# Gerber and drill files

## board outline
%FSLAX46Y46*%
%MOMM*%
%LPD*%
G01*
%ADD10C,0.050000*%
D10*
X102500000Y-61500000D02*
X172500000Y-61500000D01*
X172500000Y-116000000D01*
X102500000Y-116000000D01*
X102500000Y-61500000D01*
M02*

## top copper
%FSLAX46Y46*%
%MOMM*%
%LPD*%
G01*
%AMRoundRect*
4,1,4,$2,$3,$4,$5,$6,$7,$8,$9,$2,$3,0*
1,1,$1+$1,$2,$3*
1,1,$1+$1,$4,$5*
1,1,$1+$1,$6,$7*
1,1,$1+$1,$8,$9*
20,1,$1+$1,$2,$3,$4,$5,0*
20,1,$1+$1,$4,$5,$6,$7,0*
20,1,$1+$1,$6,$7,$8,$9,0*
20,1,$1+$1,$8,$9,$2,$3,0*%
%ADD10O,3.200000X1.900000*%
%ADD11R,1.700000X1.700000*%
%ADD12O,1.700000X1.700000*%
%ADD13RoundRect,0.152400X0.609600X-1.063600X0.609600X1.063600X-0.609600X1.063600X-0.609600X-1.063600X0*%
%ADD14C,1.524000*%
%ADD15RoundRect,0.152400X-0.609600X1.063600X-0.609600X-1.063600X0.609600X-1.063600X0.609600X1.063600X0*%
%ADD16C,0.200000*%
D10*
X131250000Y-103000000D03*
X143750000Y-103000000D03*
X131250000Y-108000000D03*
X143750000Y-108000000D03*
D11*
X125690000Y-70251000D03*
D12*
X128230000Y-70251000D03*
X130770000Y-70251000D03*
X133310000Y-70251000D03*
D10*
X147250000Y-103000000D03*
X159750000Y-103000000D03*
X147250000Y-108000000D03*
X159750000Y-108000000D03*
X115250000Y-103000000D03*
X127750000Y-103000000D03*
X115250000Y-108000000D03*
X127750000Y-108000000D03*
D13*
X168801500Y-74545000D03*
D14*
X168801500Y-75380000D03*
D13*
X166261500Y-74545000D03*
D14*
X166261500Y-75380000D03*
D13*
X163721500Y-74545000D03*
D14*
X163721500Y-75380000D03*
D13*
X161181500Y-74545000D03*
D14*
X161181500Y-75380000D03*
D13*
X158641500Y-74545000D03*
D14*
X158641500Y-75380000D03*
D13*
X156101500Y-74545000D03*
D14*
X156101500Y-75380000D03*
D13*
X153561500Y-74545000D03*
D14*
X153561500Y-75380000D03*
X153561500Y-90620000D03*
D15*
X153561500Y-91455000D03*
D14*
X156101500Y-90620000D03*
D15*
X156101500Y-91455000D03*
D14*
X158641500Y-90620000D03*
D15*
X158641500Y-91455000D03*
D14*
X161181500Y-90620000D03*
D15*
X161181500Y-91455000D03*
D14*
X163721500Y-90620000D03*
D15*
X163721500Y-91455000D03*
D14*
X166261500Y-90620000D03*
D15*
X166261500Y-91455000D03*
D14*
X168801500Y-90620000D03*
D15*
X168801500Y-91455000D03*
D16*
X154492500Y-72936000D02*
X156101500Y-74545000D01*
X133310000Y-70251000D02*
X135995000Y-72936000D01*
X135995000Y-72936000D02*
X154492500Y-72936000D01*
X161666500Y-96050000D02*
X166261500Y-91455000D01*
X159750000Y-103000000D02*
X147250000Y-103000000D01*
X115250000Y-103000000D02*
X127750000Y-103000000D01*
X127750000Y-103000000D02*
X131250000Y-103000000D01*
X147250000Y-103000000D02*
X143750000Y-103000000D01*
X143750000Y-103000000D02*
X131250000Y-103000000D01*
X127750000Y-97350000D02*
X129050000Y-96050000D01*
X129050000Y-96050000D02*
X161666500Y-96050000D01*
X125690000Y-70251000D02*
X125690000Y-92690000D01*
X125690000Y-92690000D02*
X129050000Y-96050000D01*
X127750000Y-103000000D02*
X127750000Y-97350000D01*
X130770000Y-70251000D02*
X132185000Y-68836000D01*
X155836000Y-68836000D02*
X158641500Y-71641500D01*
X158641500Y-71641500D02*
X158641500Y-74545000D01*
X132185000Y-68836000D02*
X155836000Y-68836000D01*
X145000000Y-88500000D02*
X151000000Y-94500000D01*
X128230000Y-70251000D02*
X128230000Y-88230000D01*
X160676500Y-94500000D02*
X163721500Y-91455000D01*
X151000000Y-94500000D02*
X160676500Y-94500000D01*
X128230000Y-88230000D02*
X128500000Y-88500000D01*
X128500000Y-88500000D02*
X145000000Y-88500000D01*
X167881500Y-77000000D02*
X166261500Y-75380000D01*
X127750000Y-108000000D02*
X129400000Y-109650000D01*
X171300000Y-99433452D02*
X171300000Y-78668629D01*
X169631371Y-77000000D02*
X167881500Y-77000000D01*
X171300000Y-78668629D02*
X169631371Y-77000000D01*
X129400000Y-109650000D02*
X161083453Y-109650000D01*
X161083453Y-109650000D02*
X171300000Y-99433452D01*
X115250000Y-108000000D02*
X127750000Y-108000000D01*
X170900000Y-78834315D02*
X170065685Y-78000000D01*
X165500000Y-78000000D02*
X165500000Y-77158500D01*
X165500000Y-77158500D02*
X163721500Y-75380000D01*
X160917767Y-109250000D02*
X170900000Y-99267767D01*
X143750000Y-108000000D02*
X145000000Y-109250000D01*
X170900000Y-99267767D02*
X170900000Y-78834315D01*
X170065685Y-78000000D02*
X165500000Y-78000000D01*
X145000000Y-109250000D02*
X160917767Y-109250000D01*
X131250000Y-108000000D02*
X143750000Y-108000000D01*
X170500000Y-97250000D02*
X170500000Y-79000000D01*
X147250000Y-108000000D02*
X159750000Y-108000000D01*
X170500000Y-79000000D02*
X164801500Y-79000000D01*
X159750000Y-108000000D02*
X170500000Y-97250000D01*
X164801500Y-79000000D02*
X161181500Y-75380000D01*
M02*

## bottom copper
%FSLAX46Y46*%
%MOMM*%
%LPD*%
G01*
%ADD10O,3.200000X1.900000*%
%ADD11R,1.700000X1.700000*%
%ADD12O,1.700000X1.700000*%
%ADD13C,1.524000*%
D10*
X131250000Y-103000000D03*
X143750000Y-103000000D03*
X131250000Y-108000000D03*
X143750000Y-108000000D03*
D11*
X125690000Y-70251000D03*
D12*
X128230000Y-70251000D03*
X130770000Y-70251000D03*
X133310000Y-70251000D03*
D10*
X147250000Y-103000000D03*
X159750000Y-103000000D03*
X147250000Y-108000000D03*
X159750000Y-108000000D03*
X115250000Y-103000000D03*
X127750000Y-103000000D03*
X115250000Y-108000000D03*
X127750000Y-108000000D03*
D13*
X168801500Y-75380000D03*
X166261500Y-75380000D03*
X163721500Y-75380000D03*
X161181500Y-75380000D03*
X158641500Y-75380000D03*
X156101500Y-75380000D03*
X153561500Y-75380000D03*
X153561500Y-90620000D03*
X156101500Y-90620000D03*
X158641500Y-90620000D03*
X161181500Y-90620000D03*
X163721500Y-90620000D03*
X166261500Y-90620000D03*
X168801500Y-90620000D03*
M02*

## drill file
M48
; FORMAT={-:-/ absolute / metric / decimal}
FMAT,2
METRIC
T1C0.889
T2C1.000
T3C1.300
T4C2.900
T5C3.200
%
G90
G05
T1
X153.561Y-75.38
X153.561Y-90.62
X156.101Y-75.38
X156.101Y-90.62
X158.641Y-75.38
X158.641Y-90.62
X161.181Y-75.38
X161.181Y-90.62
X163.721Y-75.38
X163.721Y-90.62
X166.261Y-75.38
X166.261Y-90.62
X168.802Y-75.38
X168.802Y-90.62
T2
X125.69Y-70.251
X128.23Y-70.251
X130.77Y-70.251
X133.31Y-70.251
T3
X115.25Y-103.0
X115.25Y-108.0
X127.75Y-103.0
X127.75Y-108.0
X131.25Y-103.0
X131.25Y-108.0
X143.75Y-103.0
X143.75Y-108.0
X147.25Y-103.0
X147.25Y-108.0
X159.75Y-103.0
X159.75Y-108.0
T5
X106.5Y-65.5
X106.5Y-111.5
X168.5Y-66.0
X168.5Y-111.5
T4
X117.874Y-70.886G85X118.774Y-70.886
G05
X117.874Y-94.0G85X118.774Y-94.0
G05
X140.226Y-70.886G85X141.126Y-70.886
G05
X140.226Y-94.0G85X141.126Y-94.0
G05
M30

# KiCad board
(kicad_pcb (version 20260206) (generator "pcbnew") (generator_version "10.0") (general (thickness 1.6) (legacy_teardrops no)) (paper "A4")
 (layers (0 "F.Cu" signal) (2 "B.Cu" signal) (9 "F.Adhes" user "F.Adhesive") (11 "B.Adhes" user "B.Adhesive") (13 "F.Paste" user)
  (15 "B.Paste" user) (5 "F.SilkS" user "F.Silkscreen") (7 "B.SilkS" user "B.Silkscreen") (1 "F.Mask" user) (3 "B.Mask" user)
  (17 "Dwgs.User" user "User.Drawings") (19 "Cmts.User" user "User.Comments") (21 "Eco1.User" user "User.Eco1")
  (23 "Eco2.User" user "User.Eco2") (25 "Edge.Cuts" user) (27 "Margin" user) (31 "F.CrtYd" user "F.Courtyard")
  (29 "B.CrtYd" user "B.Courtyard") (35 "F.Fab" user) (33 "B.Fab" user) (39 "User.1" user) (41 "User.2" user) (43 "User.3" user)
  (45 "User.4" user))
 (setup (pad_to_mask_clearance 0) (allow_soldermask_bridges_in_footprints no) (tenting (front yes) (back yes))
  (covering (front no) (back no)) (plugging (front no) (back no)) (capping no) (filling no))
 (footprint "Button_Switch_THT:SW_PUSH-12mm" (layer "F.Cu") (at 131.25 103)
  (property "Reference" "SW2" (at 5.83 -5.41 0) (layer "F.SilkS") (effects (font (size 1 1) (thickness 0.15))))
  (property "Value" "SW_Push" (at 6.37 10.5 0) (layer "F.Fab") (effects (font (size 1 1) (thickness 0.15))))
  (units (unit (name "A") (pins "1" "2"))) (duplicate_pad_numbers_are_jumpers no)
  (pad "1" thru_hole oval (at 0 0) (size 3.2 1.9) (drill 1.3) (layers "*.Cu" "*.Mask") (remove_unused_layers no) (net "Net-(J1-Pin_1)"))
  (pad "1" thru_hole oval (at 12.5 0) (size 3.2 1.9) (drill 1.3) (layers "*.Cu" "*.Mask") (remove_unused_layers no) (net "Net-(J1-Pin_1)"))
  (pad "2" thru_hole oval (at 0 5) (size 3.2 1.9) (drill 1.3) (layers "*.Cu" "*.Mask") (remove_unused_layers no) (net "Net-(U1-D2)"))
  (pad "2" thru_hole oval (at 12.5 5) (size 3.2 1.9) (drill 1.3) (layers "*.Cu" "*.Mask") (remove_unused_layers no) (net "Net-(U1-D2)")))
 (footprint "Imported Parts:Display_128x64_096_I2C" (layer "F.Cu") (at 129.5 70.251)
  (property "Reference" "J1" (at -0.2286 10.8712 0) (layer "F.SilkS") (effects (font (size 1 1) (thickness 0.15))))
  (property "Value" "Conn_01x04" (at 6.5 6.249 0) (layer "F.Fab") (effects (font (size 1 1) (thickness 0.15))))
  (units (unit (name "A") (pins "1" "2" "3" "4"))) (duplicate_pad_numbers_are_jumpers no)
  (pad "" np_thru_hole oval (at -11.176 0.635) (size 3.8 2.9) (drill oval 3.8 2.9) (layers "*.Cu" "*.Mask"))
  (pad "" np_thru_hole oval (at -11.176 23.749) (size 3.8 2.9) (drill oval 3.8 2.9) (layers "*.Cu" "*.Mask"))
  (pad "" np_thru_hole oval (at 11.176 0.635) (size 3.8 2.9) (drill oval 3.8 2.9) (layers "*.Cu" "*.Mask"))
  (pad "" np_thru_hole oval (at 11.176 23.749) (size 3.8 2.9) (drill oval 3.8 2.9) (layers "*.Cu" "*.Mask"))
  (pad "1" thru_hole rect (at -3.81 0 90) (size 1.7 1.7) (drill 1) (layers "*.Cu" "*.Mask") (remove_unused_layers no) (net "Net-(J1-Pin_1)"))
  (pad "2" thru_hole oval (at -1.27 0 90) (size 1.7 1.7) (drill 1) (layers "*.Cu" "*.Mask") (remove_unused_layers no) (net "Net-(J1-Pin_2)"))
  (pad "3" thru_hole oval (at 1.27 0 90) (size 1.7 1.7) (drill 1) (layers "*.Cu" "*.Mask") (remove_unused_layers no) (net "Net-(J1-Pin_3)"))
  (pad "4" thru_hole oval (at 3.81 0 90) (size 1.7 1.7) (drill 1) (layers "*.Cu" "*.Mask") (remove_unused_layers no) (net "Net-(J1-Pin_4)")))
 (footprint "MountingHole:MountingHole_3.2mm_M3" (layer "F.Cu") (at 168.5 66)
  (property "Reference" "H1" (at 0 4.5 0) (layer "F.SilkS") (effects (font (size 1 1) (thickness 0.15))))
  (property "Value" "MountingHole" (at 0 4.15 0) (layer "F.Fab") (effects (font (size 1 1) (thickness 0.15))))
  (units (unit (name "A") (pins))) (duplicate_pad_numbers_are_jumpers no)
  (pad "" np_thru_hole circle (at 0 0) (size 3.2 3.2) (drill 3.2) (layers "*.Cu" "*.Mask")))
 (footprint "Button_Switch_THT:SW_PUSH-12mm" (layer "F.Cu") (at 147.25 103)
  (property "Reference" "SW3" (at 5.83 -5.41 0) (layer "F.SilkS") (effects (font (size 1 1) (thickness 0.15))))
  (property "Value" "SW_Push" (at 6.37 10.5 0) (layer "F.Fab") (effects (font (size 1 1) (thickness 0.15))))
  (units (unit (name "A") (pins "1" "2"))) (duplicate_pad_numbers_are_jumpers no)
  (pad "1" thru_hole oval (at 0 0) (size 3.2 1.9) (drill 1.3) (layers "*.Cu" "*.Mask") (remove_unused_layers no) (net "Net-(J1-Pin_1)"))
  (pad "1" thru_hole oval (at 12.5 0) (size 3.2 1.9) (drill 1.3) (layers "*.Cu" "*.Mask") (remove_unused_layers no) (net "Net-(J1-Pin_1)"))
  (pad "2" thru_hole oval (at 0 5) (size 3.2 1.9) (drill 1.3) (layers "*.Cu" "*.Mask") (remove_unused_layers no) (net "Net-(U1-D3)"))
  (pad "2" thru_hole oval (at 12.5 5) (size 3.2 1.9) (drill 1.3) (layers "*.Cu" "*.Mask") (remove_unused_layers no) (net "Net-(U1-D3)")))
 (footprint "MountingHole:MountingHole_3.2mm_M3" (layer "F.Cu") (at 168.5 111.5)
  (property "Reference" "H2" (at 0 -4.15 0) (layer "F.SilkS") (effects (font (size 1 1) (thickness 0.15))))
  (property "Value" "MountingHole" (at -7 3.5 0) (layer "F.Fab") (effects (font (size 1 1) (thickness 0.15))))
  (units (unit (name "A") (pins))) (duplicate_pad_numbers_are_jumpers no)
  (pad "" np_thru_hole circle (at 0 0) (size 3.2 3.2) (drill 3.2) (layers "*.Cu" "*.Mask")))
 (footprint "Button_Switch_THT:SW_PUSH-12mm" (layer "F.Cu") (at 115.25 103)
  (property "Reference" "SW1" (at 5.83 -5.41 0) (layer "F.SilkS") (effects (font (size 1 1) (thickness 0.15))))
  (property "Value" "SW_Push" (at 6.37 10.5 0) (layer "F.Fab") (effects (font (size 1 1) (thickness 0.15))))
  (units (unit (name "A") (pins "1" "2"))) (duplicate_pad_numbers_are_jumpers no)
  (pad "1" thru_hole oval (at 0 0) (size 3.2 1.9) (drill 1.3) (layers "*.Cu" "*.Mask") (remove_unused_layers no) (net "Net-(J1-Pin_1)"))
  (pad "1" thru_hole oval (at 12.5 0) (size 3.2 1.9) (drill 1.3) (layers "*.Cu" "*.Mask") (remove_unused_layers no) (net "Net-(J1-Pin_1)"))
  (pad "2" thru_hole oval (at 0 5) (size 3.2 1.9) (drill 1.3) (layers "*.Cu" "*.Mask") (remove_unused_layers no) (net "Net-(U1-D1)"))
  (pad "2" thru_hole oval (at 12.5 5) (size 3.2 1.9) (drill 1.3) (layers "*.Cu" "*.Mask") (remove_unused_layers no) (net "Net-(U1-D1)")))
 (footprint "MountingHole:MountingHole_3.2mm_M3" (layer "F.Cu") (at 106.5 65.5)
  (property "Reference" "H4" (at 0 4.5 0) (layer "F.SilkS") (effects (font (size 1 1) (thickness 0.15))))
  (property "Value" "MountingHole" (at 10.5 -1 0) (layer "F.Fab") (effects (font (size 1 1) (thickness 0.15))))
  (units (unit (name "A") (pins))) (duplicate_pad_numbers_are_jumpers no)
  (pad "" np_thru_hole circle (at 0 0) (size 3.2 3.2) (drill 3.2) (layers "*.Cu" "*.Mask")))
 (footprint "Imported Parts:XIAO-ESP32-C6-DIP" (layer "F.Cu") (at 161.1815 83)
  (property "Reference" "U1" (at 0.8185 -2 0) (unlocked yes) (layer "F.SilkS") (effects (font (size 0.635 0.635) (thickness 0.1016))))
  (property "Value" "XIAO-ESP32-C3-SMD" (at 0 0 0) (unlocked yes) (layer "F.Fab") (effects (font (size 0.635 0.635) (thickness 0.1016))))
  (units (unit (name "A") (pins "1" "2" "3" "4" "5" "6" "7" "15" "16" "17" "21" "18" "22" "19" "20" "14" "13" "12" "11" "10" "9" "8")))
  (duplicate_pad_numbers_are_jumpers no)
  (pad "1" smd roundrect (at 7.62 -8.455 90) (size 2.432 1.524) (layers "F.Cu" "F.Mask") (roundrect_rratio 0.1)
   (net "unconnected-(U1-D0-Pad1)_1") (thermal_bridge_angle 45))
  (pad "1" thru_hole circle (at 7.62 -7.62 90) (size 1.524 1.524) (drill 0.889) (layers "*.Cu" "*.Mask") (remove_unused_layers no)
   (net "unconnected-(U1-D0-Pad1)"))
  (pad "2" smd roundrect (at 5.08 -8.455 90) (size 2.432 1.524) (layers "F.Cu" "F.Mask") (roundrect_rratio 0.1) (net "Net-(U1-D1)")
   (thermal_bridge_angle 45))
  (pad "2" thru_hole circle (at 5.08 -7.62 90) (size 1.524 1.524) (drill 0.889) (layers "*.Cu" "*.Mask") (remove_unused_layers no)
   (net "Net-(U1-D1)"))
  (pad "3" smd roundrect (at 2.54 -8.455 90) (size 2.432 1.524) (layers "F.Cu" "F.Mask") (roundrect_rratio 0.1) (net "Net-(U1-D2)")
   (thermal_bridge_angle 45))
  (pad "3" thru_hole circle (at 2.54 -7.62 90) (size 1.524 1.524) (drill 0.889) (layers "*.Cu" "*.Mask") (remove_unused_layers no)
   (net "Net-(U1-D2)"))
  (pad "4" smd roundrect (at 0 -8.455 90) (size 2.432 1.524) (layers "F.Cu" "F.Mask") (roundrect_rratio 0.1) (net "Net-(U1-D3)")
   (thermal_bridge_angle 45))
  (pad "4" thru_hole circle (at 0 -7.62 90) (size 1.524 1.524) (drill 0.889) (layers "*.Cu" "*.Mask") (remove_unused_layers no)
   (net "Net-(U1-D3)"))
  (pad "5" smd roundrect (at -2.54 -8.455 90) (size 2.432 1.524) (layers "F.Cu" "F.Mask") (roundrect_rratio 0.1) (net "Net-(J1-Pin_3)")
   (thermal_bridge_angle 45))
  (pad "5" thru_hole circle (at -2.54 -7.62 90) (size 1.524 1.524) (drill 0.889) (layers "*.Cu" "*.Mask") (remove_unused_layers no)
   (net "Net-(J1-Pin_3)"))
  (pad "6" smd roundrect (at -5.08 -8.455 90) (size 2.432 1.524) (layers "F.Cu" "F.Mask") (roundrect_rratio 0.1) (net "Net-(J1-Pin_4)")
   (thermal_bridge_angle 45))
  (pad "6" thru_hole circle (at -5.08 -7.62 90) (size 1.524 1.524) (drill 0.889) (layers "*.Cu" "*.Mask") (remove_unused_layers no)
   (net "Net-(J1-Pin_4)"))
  (pad "7" smd roundrect (at -7.62 -8.455 90) (size 2.432 1.524) (layers "F.Cu" "F.Mask") (roundrect_rratio 0.1)
   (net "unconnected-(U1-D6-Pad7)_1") (thermal_bridge_angle 45))
  (pad "7" thru_hole circle (at -7.62 -7.62 90) (size 1.524 1.524) (drill 0.889) (layers "*.Cu" "*.Mask") (remove_unused_layers no)
   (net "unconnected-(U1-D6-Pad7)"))
  (pad "8" thru_hole circle (at -7.62 7.62 270) (size 1.524 1.524) (drill 0.889) (layers "*.Cu" "*.Mask") (remove_unused_layers no)
   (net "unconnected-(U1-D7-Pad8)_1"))
  (pad "8" smd roundrect (at -7.62 8.455 270) (size 2.432 1.524) (layers "F.Cu" "F.Mask") (roundrect_rratio 0.1)
   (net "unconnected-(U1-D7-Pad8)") (thermal_bridge_angle 45))
  (pad "9" thru_hole circle (at -5.08 7.62 270) (size 1.524 1.524) (drill 0.889) (layers "*.Cu" "*.Mask") (remove_unused_layers no)
   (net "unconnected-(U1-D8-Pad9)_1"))
  (pad "9" smd roundrect (at -5.08 8.455 270) (size 2.432 1.524) (layers "F.Cu" "F.Mask") (roundrect_rratio 0.1)
   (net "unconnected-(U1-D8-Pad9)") (thermal_bridge_angle 45))
  (pad "10" thru_hole circle (at -2.54 7.62 270) (size 1.524 1.524) (drill 0.889) (layers "*.Cu" "*.Mask") (remove_unused_layers no)
   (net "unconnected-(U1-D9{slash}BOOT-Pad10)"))
  (pad "10" smd roundrect (at -2.54 8.455 270) (size 2.432 1.524) (layers "F.Cu" "F.Mask") (roundrect_rratio 0.1)
   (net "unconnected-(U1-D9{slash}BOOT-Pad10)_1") (thermal_bridge_angle 45))
  (pad "11" thru_hole circle (at 0 7.62 270) (size 1.524 1.524) (drill 0.889) (layers "*.Cu" "*.Mask") (remove_unused_layers no)
   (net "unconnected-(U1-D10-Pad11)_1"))
  (pad "11" smd roundrect (at 0 8.455 270) (size 2.432 1.524) (layers "F.Cu" "F.Mask") (roundrect_rratio 0.1)
   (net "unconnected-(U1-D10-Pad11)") (thermal_bridge_angle 45))
  (pad "12" thru_hole circle (at 2.54 7.62 270) (size 1.524 1.524) (drill 0.889) (layers "*.Cu" "*.Mask") (remove_unused_layers no)
   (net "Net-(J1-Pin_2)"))
  (pad "12" smd roundrect (at 2.54 8.455 270) (size 2.432 1.524) (layers "F.Cu" "F.Mask") (roundrect_rratio 0.1) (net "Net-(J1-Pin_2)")
   (thermal_bridge_angle 45))
  (pad "13" thru_hole circle (at 5.08 7.62 270) (size 1.524 1.524) (drill 0.889) (layers "*.Cu" "*.Mask") (remove_unused_layers no)
   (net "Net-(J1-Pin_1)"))
  (pad "13" smd roundrect (at 5.08 8.455 270) (size 2.432 1.524) (layers "F.Cu" "F.Mask") (roundrect_rratio 0.1) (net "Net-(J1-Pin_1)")
   (thermal_bridge_angle 45))
  (pad "14" thru_hole circle (at 7.62 7.62 270) (size 1.524 1.524) (drill 0.889) (layers "*.Cu" "*.Mask") (remove_unused_layers no)
   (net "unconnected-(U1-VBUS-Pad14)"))
  (pad "14" smd roundrect (at 7.62 8.455 270) (size 2.432 1.524) (layers "F.Cu" "F.Mask") (roundrect_rratio 0.1)
   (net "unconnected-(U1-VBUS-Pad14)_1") (thermal_bridge_angle 45)))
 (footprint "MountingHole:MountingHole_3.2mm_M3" (layer "F.Cu") (at 106.5 111.5)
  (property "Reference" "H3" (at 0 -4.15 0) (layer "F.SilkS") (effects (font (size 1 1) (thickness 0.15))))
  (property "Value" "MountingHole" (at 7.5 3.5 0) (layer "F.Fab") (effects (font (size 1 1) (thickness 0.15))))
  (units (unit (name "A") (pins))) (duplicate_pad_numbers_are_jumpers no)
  (pad "" np_thru_hole circle (at 0 0) (size 3.2 3.2) (drill 3.2) (layers "*.Cu" "*.Mask")))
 (gr_rect (start 102.5 61.5) (end 172.5 116) (stroke (width 0.05) (type solid)) (fill no) (layer "Edge.Cuts"))
 (segment (start 154.4925 72.936) (end 156.1015 74.545) (width 0.2) (layer "F.Cu") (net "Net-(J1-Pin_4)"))
 (segment (start 133.31 70.251) (end 135.995 72.936) (width 0.2) (layer "F.Cu") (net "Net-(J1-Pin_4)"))
 (segment (start 135.995 72.936) (end 154.4925 72.936) (width 0.2) (layer "F.Cu") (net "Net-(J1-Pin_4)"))
 (segment (start 161.6665 96.05) (end 166.2615 91.455) (width 0.2) (layer "F.Cu") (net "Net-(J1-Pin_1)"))
 (segment (start 159.75 103) (end 147.25 103) (width 0.2) (layer "F.Cu") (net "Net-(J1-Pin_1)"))
 (segment (start 115.25 103) (end 127.75 103) (width 0.2) (layer "F.Cu") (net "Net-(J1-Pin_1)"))
 (segment (start 127.75 103) (end 131.25 103) (width 0.2) (layer "F.Cu") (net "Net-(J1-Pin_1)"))
 (segment (start 147.25 103) (end 143.75 103) (width 0.2) (layer "F.Cu") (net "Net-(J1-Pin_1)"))
 (segment (start 143.75 103) (end 131.25 103) (width 0.2) (layer "F.Cu") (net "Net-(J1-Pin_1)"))
 (segment (start 127.75 97.35) (end 129.05 96.05) (width 0.2) (layer "F.Cu") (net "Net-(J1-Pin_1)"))
 (segment (start 129.05 96.05) (end 161.6665 96.05) (width 0.2) (layer "F.Cu") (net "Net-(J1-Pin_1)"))
 (segment (start 125.69 70.251) (end 125.69 92.69) (width 0.2) (layer "F.Cu") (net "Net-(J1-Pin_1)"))
 (segment (start 125.69 92.69) (end 129.05 96.05) (width 0.2) (layer "F.Cu") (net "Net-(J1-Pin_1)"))
 (segment (start 127.75 103) (end 127.75 97.35) (width 0.2) (layer "F.Cu") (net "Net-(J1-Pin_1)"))
 (segment (start 130.77 70.251) (end 132.185 68.836) (width 0.2) (layer "F.Cu") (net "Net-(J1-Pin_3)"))
 (segment (start 155.836 68.836) (end 158.6415 71.6415) (width 0.2) (layer "F.Cu") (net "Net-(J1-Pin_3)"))
 (segment (start 158.6415 71.6415) (end 158.6415 74.545) (width 0.2) (layer "F.Cu") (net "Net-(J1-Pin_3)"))
 (segment (start 132.185 68.836) (end 155.836 68.836) (width 0.2) (layer "F.Cu") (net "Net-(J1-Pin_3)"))
 (segment (start 145 88.5) (end 151 94.5) (width 0.2) (layer "F.Cu") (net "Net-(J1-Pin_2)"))
 (segment (start 128.23 70.251) (end 128.23 88.23) (width 0.2) (layer "F.Cu") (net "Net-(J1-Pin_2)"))
 (segment (start 160.6765 94.5) (end 163.7215 91.455) (width 0.2) (layer "F.Cu") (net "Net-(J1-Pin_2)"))
 (segment (start 151 94.5) (end 160.6765 94.5) (width 0.2) (layer "F.Cu") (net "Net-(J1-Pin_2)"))
 (segment (start 128.23 88.23) (end 128.5 88.5) (width 0.2) (layer "F.Cu") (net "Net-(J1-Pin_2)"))
 (segment (start 128.5 88.5) (end 145 88.5) (width 0.2) (layer "F.Cu") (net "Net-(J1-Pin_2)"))
 (segment (start 167.8815 77) (end 166.2615 75.38) (width 0.2) (layer "F.Cu") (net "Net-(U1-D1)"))
 (segment (start 127.75 108) (end 129.4 109.65) (width 0.2) (layer "F.Cu") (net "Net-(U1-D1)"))
 (segment (start 171.3 99.433452) (end 171.3 78.668629) (width 0.2) (layer "F.Cu") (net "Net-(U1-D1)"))
 (segment (start 169.631371 77) (end 167.8815 77) (width 0.2) (layer "F.Cu") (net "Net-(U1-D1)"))
 (segment (start 171.3 78.668629) (end 169.631371 77) (width 0.2) (layer "F.Cu") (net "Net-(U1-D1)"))
 (segment (start 129.4 109.65) (end 161.083453 109.65) (width 0.2) (layer "F.Cu") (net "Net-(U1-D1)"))
 (segment (start 161.083453 109.65) (end 171.3 99.433452) (width 0.2) (layer "F.Cu") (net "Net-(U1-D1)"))
 (segment (start 115.25 108) (end 127.75 108) (width 0.2) (layer "F.Cu") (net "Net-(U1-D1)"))
 (segment (start 170.9 78.834315) (end 170.065685 78) (width 0.2) (layer "F.Cu") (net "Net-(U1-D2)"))
 (segment (start 165.5 78) (end 165.5 77.1585) (width 0.2) (layer "F.Cu") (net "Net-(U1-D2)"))
 (segment (start 165.5 77.1585) (end 163.7215 75.38) (width 0.2) (layer "F.Cu") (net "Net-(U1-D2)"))
 (segment (start 160.917767 109.25) (end 170.9 99.267767) (width 0.2) (layer "F.Cu") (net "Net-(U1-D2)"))
 (segment (start 143.75 108) (end 145 109.25) (width 0.2) (layer "F.Cu") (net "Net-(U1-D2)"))
 (segment (start 170.9 99.267767) (end 170.9 78.834315) (width 0.2) (layer "F.Cu") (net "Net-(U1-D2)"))
 (segment (start 170.065685 78) (end 165.5 78) (width 0.2) (layer "F.Cu") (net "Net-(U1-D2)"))
 (segment (start 145 109.25) (end 160.917767 109.25) (width 0.2) (layer "F.Cu") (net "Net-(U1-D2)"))
 (segment (start 131.25 108) (end 143.75 108) (width 0.2) (layer "F.Cu") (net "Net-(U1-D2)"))
 (segment (start 170.5 97.25) (end 170.5 79) (width 0.2) (layer "F.Cu") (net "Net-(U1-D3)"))
 (segment (start 147.25 108) (end 159.75 108) (width 0.2) (layer "F.Cu") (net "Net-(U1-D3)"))
 (segment (start 170.5 79) (end 164.8015 79) (width 0.2) (layer "F.Cu") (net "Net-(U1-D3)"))
 (segment (start 159.75 108) (end 170.5 97.25) (width 0.2) (layer "F.Cu") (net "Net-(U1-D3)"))
 (segment (start 164.8015 79) (end 161.1815 75.38) (width 0.2) (layer "F.Cu") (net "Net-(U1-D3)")))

